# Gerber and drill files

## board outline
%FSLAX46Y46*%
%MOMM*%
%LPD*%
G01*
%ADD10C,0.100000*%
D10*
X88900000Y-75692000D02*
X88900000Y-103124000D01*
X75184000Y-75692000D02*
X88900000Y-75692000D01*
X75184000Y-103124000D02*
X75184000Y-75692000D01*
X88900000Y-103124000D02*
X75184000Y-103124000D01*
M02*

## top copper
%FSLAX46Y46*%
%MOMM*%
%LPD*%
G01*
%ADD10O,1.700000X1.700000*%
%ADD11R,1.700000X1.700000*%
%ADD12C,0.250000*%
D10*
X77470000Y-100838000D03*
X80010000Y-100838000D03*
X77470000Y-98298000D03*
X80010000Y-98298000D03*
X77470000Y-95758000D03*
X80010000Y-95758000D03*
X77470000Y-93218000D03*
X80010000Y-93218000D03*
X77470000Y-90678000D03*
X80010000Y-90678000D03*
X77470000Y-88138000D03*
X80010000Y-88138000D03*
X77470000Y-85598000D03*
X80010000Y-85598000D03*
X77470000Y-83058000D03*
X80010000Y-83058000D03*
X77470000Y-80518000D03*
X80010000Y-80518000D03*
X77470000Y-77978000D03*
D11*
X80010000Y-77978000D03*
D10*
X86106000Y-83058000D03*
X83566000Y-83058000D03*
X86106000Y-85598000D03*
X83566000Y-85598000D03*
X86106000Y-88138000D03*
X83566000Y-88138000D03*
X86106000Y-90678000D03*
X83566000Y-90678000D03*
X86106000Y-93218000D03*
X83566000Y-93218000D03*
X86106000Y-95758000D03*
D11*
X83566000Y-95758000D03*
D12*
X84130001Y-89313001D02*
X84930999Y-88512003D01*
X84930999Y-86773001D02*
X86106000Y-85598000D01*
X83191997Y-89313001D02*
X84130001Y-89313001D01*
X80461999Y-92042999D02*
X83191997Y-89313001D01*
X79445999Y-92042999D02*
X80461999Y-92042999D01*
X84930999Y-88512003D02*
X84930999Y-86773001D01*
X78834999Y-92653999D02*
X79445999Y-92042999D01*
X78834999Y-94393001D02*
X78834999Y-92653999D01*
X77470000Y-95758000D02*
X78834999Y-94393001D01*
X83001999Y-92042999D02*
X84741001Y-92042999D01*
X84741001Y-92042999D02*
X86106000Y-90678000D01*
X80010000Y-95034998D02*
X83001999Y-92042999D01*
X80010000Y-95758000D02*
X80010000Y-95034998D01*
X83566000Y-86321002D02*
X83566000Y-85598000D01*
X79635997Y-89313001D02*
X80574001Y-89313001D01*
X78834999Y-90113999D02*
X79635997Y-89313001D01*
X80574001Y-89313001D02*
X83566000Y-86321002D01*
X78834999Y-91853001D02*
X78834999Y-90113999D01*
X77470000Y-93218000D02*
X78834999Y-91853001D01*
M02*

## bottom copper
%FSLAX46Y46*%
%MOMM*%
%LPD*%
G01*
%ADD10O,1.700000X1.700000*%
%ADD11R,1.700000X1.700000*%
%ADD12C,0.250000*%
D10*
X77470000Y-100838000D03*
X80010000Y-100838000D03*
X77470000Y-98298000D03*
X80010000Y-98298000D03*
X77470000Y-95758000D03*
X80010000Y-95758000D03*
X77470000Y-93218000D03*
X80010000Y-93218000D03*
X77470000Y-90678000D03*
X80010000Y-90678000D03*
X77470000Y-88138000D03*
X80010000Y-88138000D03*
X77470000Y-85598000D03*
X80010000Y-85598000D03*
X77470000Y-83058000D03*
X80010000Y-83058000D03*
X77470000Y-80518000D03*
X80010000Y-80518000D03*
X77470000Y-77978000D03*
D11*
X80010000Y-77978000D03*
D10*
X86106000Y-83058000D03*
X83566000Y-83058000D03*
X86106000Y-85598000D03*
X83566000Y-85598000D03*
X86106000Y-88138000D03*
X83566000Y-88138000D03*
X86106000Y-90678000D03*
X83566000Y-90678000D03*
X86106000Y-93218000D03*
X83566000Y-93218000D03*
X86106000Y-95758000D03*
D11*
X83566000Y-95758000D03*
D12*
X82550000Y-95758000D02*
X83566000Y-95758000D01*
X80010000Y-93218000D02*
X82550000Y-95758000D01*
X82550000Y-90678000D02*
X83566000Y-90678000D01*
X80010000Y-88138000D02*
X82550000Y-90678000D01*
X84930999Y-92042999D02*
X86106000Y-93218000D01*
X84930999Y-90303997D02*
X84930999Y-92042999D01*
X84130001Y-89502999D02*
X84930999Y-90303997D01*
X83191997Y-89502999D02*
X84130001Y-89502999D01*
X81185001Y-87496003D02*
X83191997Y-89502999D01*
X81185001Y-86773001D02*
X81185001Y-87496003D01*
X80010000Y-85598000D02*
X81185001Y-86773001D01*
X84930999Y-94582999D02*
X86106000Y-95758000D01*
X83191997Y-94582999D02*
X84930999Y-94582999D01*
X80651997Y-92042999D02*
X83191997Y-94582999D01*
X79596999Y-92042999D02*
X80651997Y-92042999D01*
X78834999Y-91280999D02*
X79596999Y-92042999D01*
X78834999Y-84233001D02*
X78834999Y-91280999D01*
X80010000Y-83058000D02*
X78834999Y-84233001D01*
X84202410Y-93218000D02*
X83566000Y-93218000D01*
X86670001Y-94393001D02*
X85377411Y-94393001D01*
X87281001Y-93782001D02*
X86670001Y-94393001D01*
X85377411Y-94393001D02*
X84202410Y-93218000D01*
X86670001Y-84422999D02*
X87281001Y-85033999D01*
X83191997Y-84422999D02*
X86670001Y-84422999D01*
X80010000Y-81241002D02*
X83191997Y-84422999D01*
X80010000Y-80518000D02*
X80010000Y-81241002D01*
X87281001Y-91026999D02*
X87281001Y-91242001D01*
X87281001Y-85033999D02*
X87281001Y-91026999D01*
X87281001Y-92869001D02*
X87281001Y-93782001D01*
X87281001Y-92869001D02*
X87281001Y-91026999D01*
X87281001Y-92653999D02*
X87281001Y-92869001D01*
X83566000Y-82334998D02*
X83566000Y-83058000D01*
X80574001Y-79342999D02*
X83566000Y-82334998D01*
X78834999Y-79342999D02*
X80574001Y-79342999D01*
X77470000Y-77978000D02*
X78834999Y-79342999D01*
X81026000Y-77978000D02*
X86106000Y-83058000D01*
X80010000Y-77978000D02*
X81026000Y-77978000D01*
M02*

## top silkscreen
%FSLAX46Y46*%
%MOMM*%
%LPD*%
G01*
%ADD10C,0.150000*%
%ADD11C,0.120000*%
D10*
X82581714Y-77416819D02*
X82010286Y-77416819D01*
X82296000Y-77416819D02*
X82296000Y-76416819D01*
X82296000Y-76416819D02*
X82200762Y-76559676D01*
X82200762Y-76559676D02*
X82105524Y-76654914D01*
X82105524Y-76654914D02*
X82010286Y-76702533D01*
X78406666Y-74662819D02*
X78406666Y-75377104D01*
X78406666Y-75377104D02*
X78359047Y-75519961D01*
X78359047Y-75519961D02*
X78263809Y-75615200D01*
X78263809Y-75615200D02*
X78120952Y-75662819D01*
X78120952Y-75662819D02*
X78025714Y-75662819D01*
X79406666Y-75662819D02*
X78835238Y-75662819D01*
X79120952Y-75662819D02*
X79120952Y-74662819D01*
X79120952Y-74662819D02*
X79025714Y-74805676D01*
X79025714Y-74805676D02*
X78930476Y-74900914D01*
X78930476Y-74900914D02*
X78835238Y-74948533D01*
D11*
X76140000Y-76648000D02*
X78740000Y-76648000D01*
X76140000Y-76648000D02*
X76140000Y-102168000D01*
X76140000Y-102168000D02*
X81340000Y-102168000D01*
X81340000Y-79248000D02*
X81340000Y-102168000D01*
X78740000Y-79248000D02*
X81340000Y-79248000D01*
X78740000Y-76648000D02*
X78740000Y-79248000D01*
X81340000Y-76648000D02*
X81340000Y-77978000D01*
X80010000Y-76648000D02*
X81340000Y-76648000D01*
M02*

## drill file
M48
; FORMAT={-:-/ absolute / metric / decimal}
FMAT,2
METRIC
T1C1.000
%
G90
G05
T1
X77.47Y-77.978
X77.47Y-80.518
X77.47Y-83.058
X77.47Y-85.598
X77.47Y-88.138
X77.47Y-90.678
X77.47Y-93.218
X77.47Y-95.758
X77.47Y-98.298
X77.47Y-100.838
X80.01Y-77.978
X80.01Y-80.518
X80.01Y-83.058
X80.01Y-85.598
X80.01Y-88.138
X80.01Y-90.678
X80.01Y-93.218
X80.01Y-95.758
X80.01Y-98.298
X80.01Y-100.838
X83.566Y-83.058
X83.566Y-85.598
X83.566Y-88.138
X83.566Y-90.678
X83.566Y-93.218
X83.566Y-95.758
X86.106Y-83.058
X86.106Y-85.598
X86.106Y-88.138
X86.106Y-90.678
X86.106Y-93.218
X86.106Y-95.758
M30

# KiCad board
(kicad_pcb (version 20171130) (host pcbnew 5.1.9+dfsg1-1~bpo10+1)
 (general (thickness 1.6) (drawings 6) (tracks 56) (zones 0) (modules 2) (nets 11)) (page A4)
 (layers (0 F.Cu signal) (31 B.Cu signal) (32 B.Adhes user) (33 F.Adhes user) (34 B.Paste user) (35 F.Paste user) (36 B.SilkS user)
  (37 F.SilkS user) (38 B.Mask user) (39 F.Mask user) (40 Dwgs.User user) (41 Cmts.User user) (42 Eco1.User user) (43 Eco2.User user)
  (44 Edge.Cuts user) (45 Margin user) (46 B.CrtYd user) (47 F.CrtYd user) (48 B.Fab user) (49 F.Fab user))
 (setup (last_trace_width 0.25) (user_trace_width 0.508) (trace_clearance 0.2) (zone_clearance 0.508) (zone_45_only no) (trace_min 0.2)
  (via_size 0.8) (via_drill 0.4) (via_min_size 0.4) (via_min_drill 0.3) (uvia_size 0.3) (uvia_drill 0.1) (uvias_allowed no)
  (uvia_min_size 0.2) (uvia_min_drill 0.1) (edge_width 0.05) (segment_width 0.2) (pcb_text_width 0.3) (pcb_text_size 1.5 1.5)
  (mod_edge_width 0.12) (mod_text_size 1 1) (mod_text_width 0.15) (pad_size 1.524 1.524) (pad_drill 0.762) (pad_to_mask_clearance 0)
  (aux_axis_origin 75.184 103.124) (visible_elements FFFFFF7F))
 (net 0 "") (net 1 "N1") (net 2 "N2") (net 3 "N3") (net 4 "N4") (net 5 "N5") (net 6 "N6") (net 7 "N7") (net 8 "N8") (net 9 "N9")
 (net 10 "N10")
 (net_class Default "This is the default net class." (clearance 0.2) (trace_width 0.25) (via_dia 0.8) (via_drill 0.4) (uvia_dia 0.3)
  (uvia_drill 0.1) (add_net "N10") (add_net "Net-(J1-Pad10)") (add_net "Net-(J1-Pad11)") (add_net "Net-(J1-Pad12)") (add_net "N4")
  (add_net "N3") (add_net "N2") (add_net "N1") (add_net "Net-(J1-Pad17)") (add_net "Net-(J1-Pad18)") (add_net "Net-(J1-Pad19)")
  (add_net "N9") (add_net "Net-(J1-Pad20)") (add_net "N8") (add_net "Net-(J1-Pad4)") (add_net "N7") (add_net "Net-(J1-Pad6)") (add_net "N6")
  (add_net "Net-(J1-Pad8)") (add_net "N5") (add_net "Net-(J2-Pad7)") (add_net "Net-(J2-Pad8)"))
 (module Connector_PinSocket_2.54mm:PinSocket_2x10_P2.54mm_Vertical (layer F.Cu) (at 80.01 77.978)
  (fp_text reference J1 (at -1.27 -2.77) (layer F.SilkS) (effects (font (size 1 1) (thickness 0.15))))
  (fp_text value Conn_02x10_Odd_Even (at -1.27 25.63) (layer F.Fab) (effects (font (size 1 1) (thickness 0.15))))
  (fp_line (start -3.87 -1.33) (end -1.27 -1.33) (layer F.SilkS) (width 0.12))
  (fp_line (start -3.87 -1.33) (end -3.87 24.19) (layer F.SilkS) (width 0.12))
  (fp_line (start -3.87 24.19) (end 1.33 24.19) (layer F.SilkS) (width 0.12))
  (fp_line (start 1.33 1.27) (end 1.33 24.19) (layer F.SilkS) (width 0.12))
  (fp_line (start -1.27 1.27) (end 1.33 1.27) (layer F.SilkS) (width 0.12))
  (fp_line (start -1.27 -1.33) (end -1.27 1.27) (layer F.SilkS) (width 0.12))
  (fp_line (start 1.33 -1.33) (end 1.33 0) (layer F.SilkS) (width 0.12))
  (fp_line (start 0 -1.33) (end 1.33 -1.33) (layer F.SilkS) (width 0.12))
  (pad 20 thru_hole oval (at -2.54 22.86) (size 1.7 1.7) (drill 1) (layers *.Cu *.Mask))
  (pad 19 thru_hole oval (at 0 22.86) (size 1.7 1.7) (drill 1) (layers *.Cu *.Mask))
  (pad 18 thru_hole oval (at -2.54 20.32) (size 1.7 1.7) (drill 1) (layers *.Cu *.Mask))
  (pad 17 thru_hole oval (at 0 20.32) (size 1.7 1.7) (drill 1) (layers *.Cu *.Mask))
  (pad 16 thru_hole oval (at -2.54 17.78) (size 1.7 1.7) (drill 1) (layers *.Cu *.Mask) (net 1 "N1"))
  (pad 15 thru_hole oval (at 0 17.78) (size 1.7 1.7) (drill 1) (layers *.Cu *.Mask) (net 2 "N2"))
  (pad 14 thru_hole oval (at -2.54 15.24) (size 1.7 1.7) (drill 1) (layers *.Cu *.Mask) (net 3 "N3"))
  (pad 13 thru_hole oval (at 0 15.24) (size 1.7 1.7) (drill 1) (layers *.Cu *.Mask) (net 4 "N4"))
  (pad 12 thru_hole oval (at -2.54 12.7) (size 1.7 1.7) (drill 1) (layers *.Cu *.Mask))
  (pad 11 thru_hole oval (at 0 12.7) (size 1.7 1.7) (drill 1) (layers *.Cu *.Mask))
  (pad 10 thru_hole oval (at -2.54 10.16) (size 1.7 1.7) (drill 1) (layers *.Cu *.Mask))
  (pad 9 thru_hole oval (at 0 10.16) (size 1.7 1.7) (drill 1) (layers *.Cu *.Mask) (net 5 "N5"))
  (pad 8 thru_hole oval (at -2.54 7.62) (size 1.7 1.7) (drill 1) (layers *.Cu *.Mask))
  (pad 7 thru_hole oval (at 0 7.62) (size 1.7 1.7) (drill 1) (layers *.Cu *.Mask) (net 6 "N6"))
  (pad 6 thru_hole oval (at -2.54 5.08) (size 1.7 1.7) (drill 1) (layers *.Cu *.Mask))
  (pad 5 thru_hole oval (at 0 5.08) (size 1.7 1.7) (drill 1) (layers *.Cu *.Mask) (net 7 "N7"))
  (pad 4 thru_hole oval (at -2.54 2.54) (size 1.7 1.7) (drill 1) (layers *.Cu *.Mask))
  (pad 3 thru_hole oval (at 0 2.54) (size 1.7 1.7) (drill 1) (layers *.Cu *.Mask) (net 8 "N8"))
  (pad 2 thru_hole oval (at -2.54 0) (size 1.7 1.7) (drill 1) (layers *.Cu *.Mask) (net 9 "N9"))
  (pad 1 thru_hole rect (at 0 0) (size 1.7 1.7) (drill 1) (layers *.Cu *.Mask) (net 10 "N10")))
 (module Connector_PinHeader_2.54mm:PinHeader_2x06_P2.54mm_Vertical (layer B.Cu) (at 83.566 95.758)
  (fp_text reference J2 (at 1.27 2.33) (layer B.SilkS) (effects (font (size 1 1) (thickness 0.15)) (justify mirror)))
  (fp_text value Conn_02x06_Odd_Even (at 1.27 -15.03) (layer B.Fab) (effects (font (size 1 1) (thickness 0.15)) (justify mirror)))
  (pad 12 thru_hole oval (at 2.54 -12.7) (size 1.7 1.7) (drill 1) (layers *.Cu *.Mask) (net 10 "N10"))
  (pad 11 thru_hole oval (at 0 -12.7) (size 1.7 1.7) (drill 1) (layers *.Cu *.Mask) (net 9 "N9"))
  (pad 10 thru_hole oval (at 2.54 -10.16) (size 1.7 1.7) (drill 1) (layers *.Cu *.Mask) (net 1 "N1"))
  (pad 9 thru_hole oval (at 0 -10.16) (size 1.7 1.7) (drill 1) (layers *.Cu *.Mask) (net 3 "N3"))
  (pad 8 thru_hole oval (at 2.54 -7.62) (size 1.7 1.7) (drill 1) (layers *.Cu *.Mask))
  (pad 7 thru_hole oval (at 0 -7.62) (size 1.7 1.7) (drill 1) (layers *.Cu *.Mask))
  (pad 6 thru_hole oval (at 2.54 -5.08) (size 1.7 1.7) (drill 1) (layers *.Cu *.Mask) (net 2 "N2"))
  (pad 5 thru_hole oval (at 0 -5.08) (size 1.7 1.7) (drill 1) (layers *.Cu *.Mask) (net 5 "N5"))
  (pad 4 thru_hole oval (at 2.54 -2.54) (size 1.7 1.7) (drill 1) (layers *.Cu *.Mask) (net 6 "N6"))
  (pad 3 thru_hole oval (at 0 -2.54) (size 1.7 1.7) (drill 1) (layers *.Cu *.Mask) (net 8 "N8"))
  (pad 2 thru_hole oval (at 2.54 0) (size 1.7 1.7) (drill 1) (layers *.Cu *.Mask) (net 7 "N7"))
  (pad 1 thru_hole rect (at 0 0) (size 1.7 1.7) (drill 1) (layers *.Cu *.Mask) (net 4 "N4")))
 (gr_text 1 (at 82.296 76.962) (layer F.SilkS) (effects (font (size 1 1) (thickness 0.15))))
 (gr_line (start 88.9 75.692) (end 88.9 103.124) (layer Edge.Cuts) (width 0.1))
 (gr_line (start 75.184 75.692) (end 88.9 75.692) (layer Edge.Cuts) (width 0.1))
 (gr_line (start 75.184 103.124) (end 75.184 75.692) (layer Edge.Cuts) (width 0.1))
 (gr_line (start 88.9 103.124) (end 75.184 103.124) (layer Edge.Cuts) (width 0.1))
 (segment (start 84.130001 89.313001) (end 84.930999 88.512003) (width 0.25) (layer F.Cu) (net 1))
 (segment (start 84.930999 86.773001) (end 86.106 85.598) (width 0.25) (layer F.Cu) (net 1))
 (segment (start 83.191997 89.313001) (end 84.130001 89.313001) (width 0.25) (layer F.Cu) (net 1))
 (segment (start 80.461999 92.042999) (end 83.191997 89.313001) (width 0.25) (layer F.Cu) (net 1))
 (segment (start 79.445999 92.042999) (end 80.461999 92.042999) (width 0.25) (layer F.Cu) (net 1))
 (segment (start 84.930999 88.512003) (end 84.930999 86.773001) (width 0.25) (layer F.Cu) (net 1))
 (segment (start 78.834999 92.653999) (end 79.445999 92.042999) (width 0.25) (layer F.Cu) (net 1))
 (segment (start 78.834999 94.393001) (end 78.834999 92.653999) (width 0.25) (layer F.Cu) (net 1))
 (segment (start 77.47 95.758) (end 78.834999 94.393001) (width 0.25) (layer F.Cu) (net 1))
 (segment (start 83.001999 92.042999) (end 84.741001 92.042999) (width 0.25) (layer F.Cu) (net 2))
 (segment (start 84.741001 92.042999) (end 86.106 90.678) (width 0.25) (layer F.Cu) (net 2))
 (segment (start 80.01 95.034998) (end 83.001999 92.042999) (width 0.25) (layer F.Cu) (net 2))
 (segment (start 80.01 95.758) (end 80.01 95.034998) (width 0.25) (layer F.Cu) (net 2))
 (segment (start 83.566 86.321002) (end 83.566 85.598) (width 0.25) (layer F.Cu) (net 3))
 (segment (start 79.635997 89.313001) (end 80.574001 89.313001) (width 0.25) (layer F.Cu) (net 3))
 (segment (start 78.834999 90.113999) (end 79.635997 89.313001) (width 0.25) (layer F.Cu) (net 3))
 (segment (start 80.574001 89.313001) (end 83.566 86.321002) (width 0.25) (layer F.Cu) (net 3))
 (segment (start 78.834999 91.853001) (end 78.834999 90.113999) (width 0.25) (layer F.Cu) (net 3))
 (segment (start 77.47 93.218) (end 78.834999 91.853001) (width 0.25) (layer F.Cu) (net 3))
 (segment (start 82.55 95.758) (end 83.566 95.758) (width 0.25) (layer B.Cu) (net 4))
 (segment (start 80.01 93.218) (end 82.55 95.758) (width 0.25) (layer B.Cu) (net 4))
 (segment (start 82.55 90.678) (end 83.566 90.678) (width 0.25) (layer B.Cu) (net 5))
 (segment (start 80.01 88.138) (end 82.55 90.678) (width 0.25) (layer B.Cu) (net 5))
 (segment (start 84.930999 92.042999) (end 86.106 93.218) (width 0.25) (layer B.Cu) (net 6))
 (segment (start 84.930999 90.303997) (end 84.930999 92.042999) (width 0.25) (layer B.Cu) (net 6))
 (segment (start 84.130001 89.502999) (end 84.930999 90.303997) (width 0.25) (layer B.Cu) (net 6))
 (segment (start 83.191997 89.502999) (end 84.130001 89.502999) (width 0.25) (layer B.Cu) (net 6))
 (segment (start 81.185001 87.496003) (end 83.191997 89.502999) (width 0.25) (layer B.Cu) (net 6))
 (segment (start 81.185001 86.773001) (end 81.185001 87.496003) (width 0.25) (layer B.Cu) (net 6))
 (segment (start 80.01 85.598) (end 81.185001 86.773001) (width 0.25) (layer B.Cu) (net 6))
 (segment (start 84.930999 94.582999) (end 86.106 95.758) (width 0.25) (layer B.Cu) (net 7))
 (segment (start 83.191997 94.582999) (end 84.930999 94.582999) (width 0.25) (layer B.Cu) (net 7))
 (segment (start 80.651997 92.042999) (end 83.191997 94.582999) (width 0.25) (layer B.Cu) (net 7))
 (segment (start 79.596999 92.042999) (end 80.651997 92.042999) (width 0.25) (layer B.Cu) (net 7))
 (segment (start 78.834999 91.280999) (end 79.596999 92.042999) (width 0.25) (layer B.Cu) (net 7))
 (segment (start 78.834999 84.233001) (end 78.834999 91.280999) (width 0.25) (layer B.Cu) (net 7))
 (segment (start 80.01 83.058) (end 78.834999 84.233001) (width 0.25) (layer B.Cu) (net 7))
 (segment (start 84.20241 93.218) (end 83.566 93.218) (width 0.25) (layer B.Cu) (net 8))
 (segment (start 86.670001 94.393001) (end 85.377411 94.393001) (width 0.25) (layer B.Cu) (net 8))
 (segment (start 87.281001 93.782001) (end 86.670001 94.393001) (width 0.25) (layer B.Cu) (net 8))
 (segment (start 85.377411 94.393001) (end 84.20241 93.218) (width 0.25) (layer B.Cu) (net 8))
 (segment (start 86.670001 84.422999) (end 87.281001 85.033999) (width 0.25) (layer B.Cu) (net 8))
 (segment (start 83.191997 84.422999) (end 86.670001 84.422999) (width 0.25) (layer B.Cu) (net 8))
 (segment (start 80.01 81.241002) (end 83.191997 84.422999) (width 0.25) (layer B.Cu) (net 8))
 (segment (start 80.01 80.518) (end 80.01 81.241002) (width 0.25) (layer B.Cu) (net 8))
 (segment (start 87.281001 91.026999) (end 87.281001 91.242001) (width 0.25) (layer B.Cu) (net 8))
 (segment (start 87.281001 85.033999) (end 87.281001 91.026999) (width 0.25) (layer B.Cu) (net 8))
 (segment (start 87.281001 92.869001) (end 87.281001 93.782001) (width 0.25) (layer B.Cu) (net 8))
 (segment (start 87.281001 92.869001) (end 87.281001 91.026999) (width 0.25) (layer B.Cu) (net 8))
 (segment (start 87.281001 92.653999) (end 87.281001 92.869001) (width 0.25) (layer B.Cu) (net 8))
 (segment (start 83.566 82.334998) (end 83.566 83.058) (width 0.25) (layer B.Cu) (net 9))
 (segment (start 80.574001 79.342999) (end 83.566 82.334998) (width 0.25) (layer B.Cu) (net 9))
 (segment (start 78.834999 79.342999) (end 80.574001 79.342999) (width 0.25) (layer B.Cu) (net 9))
 (segment (start 77.47 77.978) (end 78.834999 79.342999) (width 0.25) (layer B.Cu) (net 9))
 (segment (start 81.026 77.978) (end 86.106 83.058) (width 0.25) (layer B.Cu) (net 10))
 (segment (start 80.01 77.978) (end 81.026 77.978) (width 0.25) (layer B.Cu) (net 10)))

